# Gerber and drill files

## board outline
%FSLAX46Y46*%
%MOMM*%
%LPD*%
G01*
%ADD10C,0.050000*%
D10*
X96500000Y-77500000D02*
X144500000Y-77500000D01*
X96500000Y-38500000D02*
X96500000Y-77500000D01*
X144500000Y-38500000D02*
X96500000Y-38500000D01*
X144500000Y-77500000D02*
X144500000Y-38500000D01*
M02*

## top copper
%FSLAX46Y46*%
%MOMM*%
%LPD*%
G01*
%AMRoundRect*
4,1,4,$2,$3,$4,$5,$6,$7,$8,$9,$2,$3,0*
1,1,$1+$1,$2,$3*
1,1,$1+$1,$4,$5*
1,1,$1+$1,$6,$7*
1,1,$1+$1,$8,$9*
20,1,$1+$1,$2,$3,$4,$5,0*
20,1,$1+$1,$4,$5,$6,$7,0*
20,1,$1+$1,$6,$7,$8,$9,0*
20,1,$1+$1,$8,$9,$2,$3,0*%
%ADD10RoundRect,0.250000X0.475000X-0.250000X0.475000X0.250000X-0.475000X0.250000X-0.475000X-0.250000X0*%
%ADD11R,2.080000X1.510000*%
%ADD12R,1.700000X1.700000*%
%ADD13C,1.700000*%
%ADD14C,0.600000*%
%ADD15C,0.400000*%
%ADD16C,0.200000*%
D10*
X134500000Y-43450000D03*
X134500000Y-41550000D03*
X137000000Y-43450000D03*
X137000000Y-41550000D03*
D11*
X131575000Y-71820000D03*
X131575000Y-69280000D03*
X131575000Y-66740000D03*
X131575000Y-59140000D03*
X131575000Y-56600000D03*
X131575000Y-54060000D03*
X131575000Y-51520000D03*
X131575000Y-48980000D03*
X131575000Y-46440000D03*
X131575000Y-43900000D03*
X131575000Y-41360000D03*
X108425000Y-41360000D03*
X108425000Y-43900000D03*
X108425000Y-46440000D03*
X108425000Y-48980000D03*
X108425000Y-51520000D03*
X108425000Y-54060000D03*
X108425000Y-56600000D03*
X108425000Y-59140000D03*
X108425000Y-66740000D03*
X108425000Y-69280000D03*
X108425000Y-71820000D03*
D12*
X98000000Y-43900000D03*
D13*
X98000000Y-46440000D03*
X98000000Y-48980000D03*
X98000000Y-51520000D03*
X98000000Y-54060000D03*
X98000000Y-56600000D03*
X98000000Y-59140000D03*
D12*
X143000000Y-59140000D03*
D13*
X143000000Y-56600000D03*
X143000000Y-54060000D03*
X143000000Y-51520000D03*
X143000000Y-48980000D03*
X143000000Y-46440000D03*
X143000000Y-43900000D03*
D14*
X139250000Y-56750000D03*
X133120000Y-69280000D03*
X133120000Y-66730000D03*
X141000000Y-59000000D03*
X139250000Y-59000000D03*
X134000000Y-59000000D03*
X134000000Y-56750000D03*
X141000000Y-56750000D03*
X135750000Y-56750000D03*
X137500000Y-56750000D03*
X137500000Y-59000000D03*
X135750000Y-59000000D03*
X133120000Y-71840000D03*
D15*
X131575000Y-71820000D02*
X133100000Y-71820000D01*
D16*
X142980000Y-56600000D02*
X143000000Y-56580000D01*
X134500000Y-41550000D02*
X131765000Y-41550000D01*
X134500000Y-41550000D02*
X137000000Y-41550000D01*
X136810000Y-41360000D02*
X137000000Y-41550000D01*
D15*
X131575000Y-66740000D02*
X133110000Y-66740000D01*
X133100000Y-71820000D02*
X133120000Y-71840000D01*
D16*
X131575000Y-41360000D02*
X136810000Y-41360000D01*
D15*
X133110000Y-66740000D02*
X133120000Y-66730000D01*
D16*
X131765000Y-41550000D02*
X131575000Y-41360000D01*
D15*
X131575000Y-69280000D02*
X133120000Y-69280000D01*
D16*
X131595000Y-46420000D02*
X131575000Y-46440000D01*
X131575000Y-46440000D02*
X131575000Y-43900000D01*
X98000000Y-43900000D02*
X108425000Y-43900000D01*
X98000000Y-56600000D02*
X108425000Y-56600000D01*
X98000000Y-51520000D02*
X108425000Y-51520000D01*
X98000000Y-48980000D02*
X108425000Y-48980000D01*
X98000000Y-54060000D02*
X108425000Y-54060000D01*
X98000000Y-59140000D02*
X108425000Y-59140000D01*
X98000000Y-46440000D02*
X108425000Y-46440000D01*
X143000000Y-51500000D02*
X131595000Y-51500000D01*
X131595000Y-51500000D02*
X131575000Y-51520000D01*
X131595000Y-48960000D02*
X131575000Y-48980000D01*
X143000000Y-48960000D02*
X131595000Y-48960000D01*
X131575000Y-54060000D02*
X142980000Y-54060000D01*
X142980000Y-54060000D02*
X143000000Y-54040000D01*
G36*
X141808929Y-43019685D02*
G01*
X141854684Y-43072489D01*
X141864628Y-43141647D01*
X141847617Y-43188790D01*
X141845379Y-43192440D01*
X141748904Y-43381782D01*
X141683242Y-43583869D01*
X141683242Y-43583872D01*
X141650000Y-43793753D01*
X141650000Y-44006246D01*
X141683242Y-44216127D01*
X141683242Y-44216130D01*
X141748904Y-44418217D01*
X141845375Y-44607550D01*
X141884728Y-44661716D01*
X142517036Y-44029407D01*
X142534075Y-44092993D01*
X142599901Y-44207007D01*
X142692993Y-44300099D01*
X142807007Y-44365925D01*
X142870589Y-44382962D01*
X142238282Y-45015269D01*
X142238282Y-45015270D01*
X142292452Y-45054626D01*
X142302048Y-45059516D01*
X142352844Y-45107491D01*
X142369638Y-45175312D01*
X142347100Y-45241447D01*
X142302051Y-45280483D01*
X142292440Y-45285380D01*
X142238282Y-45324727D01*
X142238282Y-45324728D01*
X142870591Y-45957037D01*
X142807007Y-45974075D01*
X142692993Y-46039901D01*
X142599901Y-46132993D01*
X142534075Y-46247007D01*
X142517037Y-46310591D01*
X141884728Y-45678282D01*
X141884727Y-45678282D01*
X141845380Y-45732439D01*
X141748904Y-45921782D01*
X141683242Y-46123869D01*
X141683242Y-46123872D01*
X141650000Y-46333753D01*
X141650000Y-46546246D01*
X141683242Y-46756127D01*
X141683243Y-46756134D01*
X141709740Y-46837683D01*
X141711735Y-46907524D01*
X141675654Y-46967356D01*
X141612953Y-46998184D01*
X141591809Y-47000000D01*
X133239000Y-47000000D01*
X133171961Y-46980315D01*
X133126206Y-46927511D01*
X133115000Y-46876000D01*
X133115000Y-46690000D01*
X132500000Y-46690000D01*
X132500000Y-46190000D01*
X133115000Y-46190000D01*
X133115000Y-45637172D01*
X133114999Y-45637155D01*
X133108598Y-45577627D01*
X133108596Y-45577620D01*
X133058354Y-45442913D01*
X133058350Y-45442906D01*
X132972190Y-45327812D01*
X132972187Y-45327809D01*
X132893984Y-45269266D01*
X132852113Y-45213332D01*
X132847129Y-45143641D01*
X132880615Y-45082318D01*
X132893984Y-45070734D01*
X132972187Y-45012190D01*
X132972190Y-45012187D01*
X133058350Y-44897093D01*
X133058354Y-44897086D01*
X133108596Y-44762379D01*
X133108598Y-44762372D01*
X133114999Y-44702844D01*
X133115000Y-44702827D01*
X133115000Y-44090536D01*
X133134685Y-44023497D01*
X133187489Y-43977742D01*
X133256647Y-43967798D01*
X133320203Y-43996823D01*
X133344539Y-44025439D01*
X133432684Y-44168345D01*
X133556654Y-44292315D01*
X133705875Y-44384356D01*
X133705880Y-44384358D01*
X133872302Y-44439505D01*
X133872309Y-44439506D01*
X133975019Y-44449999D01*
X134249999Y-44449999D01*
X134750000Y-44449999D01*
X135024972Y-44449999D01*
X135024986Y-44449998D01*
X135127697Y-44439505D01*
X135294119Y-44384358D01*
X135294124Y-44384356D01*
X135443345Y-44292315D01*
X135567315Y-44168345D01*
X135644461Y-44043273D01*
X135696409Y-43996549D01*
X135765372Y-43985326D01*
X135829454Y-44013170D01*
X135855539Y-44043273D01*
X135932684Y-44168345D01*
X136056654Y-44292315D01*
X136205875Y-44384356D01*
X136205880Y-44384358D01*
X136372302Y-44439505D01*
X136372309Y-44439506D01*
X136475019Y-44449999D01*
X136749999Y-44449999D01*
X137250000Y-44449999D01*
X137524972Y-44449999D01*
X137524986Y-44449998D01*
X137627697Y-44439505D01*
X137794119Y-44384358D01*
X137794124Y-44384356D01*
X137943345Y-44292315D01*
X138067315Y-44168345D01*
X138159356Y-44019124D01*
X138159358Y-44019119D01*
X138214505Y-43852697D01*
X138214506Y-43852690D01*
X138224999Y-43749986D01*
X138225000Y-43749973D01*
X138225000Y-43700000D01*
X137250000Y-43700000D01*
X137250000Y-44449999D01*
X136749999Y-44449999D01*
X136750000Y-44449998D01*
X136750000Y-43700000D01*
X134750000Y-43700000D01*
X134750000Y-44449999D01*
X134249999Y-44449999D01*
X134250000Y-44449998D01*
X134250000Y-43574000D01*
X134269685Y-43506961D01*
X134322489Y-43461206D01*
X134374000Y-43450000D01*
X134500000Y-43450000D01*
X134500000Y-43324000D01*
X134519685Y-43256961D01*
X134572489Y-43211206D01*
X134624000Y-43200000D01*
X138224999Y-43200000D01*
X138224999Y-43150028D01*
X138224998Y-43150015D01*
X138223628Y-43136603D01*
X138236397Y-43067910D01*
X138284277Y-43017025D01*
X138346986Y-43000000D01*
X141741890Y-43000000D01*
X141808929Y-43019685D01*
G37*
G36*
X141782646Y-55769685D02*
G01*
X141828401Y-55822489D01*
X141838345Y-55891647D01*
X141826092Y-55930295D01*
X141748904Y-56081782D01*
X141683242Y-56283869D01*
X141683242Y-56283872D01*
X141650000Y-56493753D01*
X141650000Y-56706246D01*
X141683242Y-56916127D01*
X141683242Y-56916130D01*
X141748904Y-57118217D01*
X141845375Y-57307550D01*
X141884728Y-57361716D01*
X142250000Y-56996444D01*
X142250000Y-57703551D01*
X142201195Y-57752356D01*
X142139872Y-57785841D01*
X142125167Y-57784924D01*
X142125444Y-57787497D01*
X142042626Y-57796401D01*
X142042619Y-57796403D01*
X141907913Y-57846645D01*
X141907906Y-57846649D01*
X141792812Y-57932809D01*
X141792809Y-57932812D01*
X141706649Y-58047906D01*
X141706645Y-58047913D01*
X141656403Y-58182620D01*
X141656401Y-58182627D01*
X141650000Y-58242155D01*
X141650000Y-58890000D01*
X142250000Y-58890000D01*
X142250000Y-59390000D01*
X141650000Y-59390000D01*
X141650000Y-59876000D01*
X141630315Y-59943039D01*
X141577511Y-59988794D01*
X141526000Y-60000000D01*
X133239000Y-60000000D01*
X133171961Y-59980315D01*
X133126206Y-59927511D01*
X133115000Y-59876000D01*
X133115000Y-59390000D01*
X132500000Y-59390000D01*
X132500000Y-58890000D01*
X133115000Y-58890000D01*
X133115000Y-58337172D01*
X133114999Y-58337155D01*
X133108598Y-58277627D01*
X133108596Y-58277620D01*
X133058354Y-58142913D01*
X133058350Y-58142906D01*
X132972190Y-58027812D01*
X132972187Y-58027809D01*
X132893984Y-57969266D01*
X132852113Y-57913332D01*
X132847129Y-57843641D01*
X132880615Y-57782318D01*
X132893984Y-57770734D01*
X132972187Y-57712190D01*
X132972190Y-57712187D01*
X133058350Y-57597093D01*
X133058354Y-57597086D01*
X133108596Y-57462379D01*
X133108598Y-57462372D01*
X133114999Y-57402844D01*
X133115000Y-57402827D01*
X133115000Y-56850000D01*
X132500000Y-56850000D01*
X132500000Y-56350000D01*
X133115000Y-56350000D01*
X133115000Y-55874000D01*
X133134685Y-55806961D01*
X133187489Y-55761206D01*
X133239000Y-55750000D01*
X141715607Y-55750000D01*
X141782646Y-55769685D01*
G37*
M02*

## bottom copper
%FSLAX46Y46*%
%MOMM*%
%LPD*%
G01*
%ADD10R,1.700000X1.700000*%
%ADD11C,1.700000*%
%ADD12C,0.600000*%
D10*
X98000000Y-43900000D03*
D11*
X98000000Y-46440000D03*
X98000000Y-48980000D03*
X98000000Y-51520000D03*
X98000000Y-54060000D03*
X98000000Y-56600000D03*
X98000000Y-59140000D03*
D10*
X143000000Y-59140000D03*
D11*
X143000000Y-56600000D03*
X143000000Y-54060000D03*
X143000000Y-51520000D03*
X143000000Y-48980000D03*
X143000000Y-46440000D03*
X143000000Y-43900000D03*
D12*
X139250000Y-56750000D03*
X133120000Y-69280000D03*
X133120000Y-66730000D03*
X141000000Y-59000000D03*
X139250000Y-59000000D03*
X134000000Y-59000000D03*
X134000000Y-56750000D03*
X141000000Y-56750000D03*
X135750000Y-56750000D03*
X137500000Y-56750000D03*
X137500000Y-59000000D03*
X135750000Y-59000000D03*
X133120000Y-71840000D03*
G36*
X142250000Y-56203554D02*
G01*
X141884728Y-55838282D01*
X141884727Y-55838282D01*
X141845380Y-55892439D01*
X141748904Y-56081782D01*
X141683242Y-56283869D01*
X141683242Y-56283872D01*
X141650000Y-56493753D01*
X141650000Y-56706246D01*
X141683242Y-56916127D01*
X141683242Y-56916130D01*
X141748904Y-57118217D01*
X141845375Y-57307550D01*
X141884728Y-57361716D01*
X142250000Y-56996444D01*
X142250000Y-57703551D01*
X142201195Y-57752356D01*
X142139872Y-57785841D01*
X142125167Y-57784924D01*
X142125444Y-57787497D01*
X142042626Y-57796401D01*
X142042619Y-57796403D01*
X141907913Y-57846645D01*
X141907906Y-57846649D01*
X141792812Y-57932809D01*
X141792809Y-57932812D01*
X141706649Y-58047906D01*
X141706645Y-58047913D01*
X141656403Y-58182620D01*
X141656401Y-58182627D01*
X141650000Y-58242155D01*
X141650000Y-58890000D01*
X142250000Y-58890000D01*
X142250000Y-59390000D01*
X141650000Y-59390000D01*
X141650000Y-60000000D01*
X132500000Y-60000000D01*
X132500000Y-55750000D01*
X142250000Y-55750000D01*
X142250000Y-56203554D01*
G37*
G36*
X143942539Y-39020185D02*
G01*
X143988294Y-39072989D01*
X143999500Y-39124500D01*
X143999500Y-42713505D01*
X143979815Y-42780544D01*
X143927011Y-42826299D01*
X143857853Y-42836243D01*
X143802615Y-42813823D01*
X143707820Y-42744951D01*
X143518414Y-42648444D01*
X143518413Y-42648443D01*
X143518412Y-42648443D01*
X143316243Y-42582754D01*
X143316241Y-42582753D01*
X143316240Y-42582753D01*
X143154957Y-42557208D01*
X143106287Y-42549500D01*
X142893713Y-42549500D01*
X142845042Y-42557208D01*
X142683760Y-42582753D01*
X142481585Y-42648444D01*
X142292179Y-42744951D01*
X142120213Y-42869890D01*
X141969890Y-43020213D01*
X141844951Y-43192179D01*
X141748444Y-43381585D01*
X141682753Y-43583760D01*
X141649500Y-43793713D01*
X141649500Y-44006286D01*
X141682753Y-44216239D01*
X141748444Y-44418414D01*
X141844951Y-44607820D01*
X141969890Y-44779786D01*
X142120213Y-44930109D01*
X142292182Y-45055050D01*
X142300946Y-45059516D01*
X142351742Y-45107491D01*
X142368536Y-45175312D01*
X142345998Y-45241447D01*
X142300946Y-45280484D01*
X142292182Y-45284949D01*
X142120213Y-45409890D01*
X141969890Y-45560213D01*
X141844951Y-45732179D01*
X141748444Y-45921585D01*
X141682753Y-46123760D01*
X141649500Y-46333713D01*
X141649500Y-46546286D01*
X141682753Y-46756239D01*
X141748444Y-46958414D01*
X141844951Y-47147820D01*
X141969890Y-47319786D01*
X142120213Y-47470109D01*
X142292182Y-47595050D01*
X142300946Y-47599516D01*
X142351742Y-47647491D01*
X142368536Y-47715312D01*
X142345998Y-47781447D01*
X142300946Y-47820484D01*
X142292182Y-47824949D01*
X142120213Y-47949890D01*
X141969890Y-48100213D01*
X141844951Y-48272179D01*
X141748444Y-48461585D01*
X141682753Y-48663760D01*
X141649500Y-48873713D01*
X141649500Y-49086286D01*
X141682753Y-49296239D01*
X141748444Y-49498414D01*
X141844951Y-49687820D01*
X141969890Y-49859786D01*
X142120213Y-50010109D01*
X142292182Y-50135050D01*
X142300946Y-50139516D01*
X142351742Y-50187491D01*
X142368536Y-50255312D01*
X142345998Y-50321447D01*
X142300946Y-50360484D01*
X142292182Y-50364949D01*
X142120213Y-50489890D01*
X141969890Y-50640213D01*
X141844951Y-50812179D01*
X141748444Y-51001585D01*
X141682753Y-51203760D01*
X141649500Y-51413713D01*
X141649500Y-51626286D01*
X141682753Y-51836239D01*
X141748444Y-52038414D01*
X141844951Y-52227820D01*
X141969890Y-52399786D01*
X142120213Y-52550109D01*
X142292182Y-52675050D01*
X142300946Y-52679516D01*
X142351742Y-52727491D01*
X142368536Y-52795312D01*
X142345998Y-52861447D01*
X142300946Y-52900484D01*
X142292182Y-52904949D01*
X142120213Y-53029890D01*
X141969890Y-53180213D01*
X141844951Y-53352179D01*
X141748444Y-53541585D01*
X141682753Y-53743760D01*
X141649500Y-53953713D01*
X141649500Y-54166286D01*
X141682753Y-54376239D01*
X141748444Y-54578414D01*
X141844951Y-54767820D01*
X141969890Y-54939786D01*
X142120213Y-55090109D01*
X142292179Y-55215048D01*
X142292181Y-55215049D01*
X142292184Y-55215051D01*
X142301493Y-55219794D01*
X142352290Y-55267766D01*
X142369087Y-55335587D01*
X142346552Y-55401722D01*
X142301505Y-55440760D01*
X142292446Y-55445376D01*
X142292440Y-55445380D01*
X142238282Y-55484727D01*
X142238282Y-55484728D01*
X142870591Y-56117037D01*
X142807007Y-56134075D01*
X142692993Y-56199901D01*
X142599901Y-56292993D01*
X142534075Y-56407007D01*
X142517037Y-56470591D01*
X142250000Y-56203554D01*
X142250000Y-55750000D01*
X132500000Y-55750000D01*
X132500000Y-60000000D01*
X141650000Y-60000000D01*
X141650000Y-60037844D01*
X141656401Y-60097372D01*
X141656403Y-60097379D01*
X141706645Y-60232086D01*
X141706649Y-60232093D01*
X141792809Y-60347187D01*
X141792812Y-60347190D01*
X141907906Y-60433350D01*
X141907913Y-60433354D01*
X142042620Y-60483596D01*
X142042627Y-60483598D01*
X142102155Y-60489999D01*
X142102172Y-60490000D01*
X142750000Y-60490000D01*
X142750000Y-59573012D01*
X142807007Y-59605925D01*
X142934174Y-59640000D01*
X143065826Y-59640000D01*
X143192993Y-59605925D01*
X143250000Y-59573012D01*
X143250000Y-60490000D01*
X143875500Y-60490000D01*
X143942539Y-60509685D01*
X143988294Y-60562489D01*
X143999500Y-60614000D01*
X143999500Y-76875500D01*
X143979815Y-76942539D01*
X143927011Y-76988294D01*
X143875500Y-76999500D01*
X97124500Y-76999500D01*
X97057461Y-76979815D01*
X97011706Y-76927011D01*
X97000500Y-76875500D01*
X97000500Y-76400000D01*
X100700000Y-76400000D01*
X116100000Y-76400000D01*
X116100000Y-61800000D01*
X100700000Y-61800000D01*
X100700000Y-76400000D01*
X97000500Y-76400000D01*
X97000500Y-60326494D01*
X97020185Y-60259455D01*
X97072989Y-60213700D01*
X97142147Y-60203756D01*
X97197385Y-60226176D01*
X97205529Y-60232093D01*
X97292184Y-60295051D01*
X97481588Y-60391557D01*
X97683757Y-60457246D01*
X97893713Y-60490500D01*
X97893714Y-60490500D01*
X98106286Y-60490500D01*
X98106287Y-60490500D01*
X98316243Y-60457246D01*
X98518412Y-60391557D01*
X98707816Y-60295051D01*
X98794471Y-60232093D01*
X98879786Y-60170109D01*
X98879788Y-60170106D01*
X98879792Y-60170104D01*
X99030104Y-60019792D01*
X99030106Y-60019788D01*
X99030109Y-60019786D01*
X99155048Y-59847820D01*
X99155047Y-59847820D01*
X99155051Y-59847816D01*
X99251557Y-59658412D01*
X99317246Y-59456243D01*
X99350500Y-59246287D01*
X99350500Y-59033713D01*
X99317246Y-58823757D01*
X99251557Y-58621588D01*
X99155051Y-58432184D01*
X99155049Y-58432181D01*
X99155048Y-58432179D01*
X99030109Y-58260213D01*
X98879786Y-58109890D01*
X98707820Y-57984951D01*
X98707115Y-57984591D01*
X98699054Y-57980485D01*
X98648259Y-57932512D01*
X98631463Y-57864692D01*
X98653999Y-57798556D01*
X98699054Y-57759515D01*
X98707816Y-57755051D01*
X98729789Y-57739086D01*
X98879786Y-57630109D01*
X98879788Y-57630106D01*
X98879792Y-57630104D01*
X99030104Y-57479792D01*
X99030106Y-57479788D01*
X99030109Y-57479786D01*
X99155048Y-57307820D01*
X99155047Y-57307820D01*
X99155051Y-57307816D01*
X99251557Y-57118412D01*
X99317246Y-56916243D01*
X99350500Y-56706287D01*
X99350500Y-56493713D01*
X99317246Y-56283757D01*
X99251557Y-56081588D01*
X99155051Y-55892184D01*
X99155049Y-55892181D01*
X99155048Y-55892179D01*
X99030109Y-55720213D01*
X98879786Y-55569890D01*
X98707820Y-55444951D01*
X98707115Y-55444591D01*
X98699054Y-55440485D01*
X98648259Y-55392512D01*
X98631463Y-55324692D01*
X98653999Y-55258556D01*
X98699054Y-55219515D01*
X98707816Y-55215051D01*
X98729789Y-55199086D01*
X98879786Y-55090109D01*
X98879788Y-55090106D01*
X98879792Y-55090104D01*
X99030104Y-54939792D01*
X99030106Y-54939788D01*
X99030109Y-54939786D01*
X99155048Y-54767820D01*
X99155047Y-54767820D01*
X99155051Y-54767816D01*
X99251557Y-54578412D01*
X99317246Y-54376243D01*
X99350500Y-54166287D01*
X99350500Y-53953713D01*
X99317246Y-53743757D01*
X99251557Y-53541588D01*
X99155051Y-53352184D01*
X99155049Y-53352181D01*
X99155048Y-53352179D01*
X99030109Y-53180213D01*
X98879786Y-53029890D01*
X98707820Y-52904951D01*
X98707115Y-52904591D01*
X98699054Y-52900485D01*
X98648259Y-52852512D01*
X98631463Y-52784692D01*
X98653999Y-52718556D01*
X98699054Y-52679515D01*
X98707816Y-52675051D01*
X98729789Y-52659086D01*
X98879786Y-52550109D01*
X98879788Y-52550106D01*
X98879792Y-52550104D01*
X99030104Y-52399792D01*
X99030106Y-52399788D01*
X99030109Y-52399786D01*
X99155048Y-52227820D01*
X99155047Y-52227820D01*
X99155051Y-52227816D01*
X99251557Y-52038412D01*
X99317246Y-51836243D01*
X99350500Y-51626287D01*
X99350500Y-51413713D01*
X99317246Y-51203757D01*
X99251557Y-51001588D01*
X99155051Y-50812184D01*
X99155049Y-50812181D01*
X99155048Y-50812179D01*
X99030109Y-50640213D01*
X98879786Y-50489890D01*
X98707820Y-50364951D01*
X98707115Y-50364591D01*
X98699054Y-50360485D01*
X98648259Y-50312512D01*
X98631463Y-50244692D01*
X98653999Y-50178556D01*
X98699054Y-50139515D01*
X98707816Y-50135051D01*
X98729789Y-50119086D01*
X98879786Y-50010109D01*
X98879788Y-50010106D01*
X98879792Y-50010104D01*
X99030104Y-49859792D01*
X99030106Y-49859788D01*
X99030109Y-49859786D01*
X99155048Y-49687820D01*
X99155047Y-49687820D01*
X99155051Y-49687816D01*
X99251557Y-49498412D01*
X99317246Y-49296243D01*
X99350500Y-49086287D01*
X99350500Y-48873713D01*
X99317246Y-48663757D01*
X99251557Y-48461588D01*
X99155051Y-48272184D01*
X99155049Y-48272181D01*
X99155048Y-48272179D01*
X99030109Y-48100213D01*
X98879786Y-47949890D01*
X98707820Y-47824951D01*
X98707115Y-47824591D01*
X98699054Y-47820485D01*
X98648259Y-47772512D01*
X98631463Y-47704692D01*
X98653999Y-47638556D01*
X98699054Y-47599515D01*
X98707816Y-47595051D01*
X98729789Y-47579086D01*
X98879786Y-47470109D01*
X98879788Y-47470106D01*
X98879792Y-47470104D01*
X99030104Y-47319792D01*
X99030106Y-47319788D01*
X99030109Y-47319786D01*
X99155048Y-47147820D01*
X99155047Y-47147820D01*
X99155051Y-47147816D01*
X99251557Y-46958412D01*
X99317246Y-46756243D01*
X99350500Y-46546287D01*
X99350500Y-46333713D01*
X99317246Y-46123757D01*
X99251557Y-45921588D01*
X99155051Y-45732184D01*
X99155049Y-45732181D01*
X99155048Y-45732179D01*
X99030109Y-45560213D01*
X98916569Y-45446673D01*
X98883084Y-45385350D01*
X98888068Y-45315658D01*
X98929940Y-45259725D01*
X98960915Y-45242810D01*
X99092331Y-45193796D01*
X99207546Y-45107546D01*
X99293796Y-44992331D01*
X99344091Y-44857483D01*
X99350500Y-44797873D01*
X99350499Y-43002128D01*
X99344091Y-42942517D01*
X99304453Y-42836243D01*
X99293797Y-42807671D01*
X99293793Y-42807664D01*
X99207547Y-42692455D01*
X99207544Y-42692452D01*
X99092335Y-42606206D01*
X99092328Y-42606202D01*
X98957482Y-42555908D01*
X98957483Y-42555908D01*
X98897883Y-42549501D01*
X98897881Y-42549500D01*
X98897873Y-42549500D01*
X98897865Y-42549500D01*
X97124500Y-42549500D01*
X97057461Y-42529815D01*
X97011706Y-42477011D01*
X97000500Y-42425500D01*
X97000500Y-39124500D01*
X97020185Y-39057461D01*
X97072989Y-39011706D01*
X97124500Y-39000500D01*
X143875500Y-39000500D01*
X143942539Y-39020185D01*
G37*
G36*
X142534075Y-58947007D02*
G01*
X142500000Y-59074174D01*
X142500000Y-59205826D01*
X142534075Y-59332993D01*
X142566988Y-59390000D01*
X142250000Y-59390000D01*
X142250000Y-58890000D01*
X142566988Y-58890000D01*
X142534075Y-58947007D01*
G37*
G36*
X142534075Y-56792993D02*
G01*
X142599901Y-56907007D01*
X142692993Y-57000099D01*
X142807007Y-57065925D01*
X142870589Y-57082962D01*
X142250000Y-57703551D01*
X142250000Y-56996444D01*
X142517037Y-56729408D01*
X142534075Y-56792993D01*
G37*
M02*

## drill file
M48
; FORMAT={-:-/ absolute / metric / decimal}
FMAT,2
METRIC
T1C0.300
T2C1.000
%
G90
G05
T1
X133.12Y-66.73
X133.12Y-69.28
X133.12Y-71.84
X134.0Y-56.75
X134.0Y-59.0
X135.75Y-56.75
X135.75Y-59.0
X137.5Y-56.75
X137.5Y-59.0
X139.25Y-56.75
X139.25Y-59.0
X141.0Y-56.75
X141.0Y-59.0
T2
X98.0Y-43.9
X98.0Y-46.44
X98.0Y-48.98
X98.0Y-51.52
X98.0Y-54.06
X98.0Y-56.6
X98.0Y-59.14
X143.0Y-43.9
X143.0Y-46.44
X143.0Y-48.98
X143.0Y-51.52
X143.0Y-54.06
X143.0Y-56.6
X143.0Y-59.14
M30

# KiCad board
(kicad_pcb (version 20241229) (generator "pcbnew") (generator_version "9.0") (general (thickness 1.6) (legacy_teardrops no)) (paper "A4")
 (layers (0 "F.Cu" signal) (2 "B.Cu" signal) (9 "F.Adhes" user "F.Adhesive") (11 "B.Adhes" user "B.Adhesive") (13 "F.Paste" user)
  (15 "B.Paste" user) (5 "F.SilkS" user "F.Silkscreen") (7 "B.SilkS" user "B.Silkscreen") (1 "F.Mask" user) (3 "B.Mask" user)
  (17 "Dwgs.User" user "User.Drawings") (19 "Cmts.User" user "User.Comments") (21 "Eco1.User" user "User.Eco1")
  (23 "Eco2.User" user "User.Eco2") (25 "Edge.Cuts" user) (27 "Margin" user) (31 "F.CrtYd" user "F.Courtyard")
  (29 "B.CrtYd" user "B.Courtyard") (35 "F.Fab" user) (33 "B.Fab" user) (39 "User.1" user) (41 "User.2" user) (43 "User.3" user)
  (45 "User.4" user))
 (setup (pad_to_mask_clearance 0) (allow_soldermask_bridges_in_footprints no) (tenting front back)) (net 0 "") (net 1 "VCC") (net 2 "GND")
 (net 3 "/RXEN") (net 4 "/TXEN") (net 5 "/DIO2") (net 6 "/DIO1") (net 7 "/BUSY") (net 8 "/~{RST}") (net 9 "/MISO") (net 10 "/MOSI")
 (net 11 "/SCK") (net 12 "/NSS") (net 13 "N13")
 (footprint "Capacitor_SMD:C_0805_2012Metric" (layer "F.Cu") (at 134.5 42.5 90)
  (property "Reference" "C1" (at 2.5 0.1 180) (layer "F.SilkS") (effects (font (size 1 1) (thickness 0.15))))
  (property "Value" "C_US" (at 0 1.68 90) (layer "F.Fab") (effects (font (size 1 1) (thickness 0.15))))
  (pad "1" smd roundrect (at -0.95 0 90) (size 1 1.45) (layers "F.Cu" "F.Mask" "F.Paste") (roundrect_rratio 0.25) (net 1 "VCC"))
  (pad "2" smd roundrect (at 0.95 0 90) (size 1 1.45) (layers "F.Cu" "F.Mask" "F.Paste") (roundrect_rratio 0.25) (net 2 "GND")))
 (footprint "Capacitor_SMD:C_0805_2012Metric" (layer "F.Cu") (at 137 42.5 90)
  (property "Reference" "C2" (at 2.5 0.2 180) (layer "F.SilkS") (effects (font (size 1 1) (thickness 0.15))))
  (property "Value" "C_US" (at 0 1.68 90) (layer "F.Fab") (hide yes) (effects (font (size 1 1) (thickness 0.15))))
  (pad "1" smd roundrect (at -0.95 0 90) (size 1 1.45) (layers "F.Cu" "F.Mask" "F.Paste") (roundrect_rratio 0.25) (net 1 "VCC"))
  (pad "2" smd roundrect (at 0.95 0 90) (size 1 1.45) (layers "F.Cu" "F.Mask" "F.Paste") (roundrect_rratio 0.25) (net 2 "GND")))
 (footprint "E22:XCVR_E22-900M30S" (layer "F.Cu") (at 120 58)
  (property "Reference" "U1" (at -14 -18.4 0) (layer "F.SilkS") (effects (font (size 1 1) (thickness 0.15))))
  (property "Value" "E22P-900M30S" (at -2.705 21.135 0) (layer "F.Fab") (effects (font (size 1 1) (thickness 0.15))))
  (pad "1" smd rect (at 11.575 13.82) (size 2.08 1.51) (layers "F.Cu" "F.Mask" "F.Paste") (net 2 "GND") (solder_mask_margin 0.102))
  (pad "2" smd rect (at 11.575 11.28) (size 2.08 1.51) (layers "F.Cu" "F.Mask" "F.Paste") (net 2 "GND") (solder_mask_margin 0.102))
  (pad "3" smd rect (at 11.575 8.74) (size 2.08 1.51) (layers "F.Cu" "F.Mask" "F.Paste") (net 2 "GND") (solder_mask_margin 0.102))
  (pad "4" smd rect (at 11.575 1.14) (size 2.08 1.51) (layers "F.Cu" "F.Mask" "F.Paste") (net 2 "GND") (solder_mask_margin 0.102))
  (pad "5" smd rect (at 11.575 -1.4) (size 2.08 1.51) (layers "F.Cu" "F.Mask" "F.Paste") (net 2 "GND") (solder_mask_margin 0.102))
  (pad "6" smd rect (at 11.575 -3.94) (size 2.08 1.51) (layers "F.Cu" "F.Mask" "F.Paste") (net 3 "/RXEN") (solder_mask_margin 0.102))
  (pad "7" smd rect (at 11.575 -6.48) (size 2.08 1.51) (layers "F.Cu" "F.Mask" "F.Paste") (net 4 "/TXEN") (solder_mask_margin 0.102))
  (pad "8" smd rect (at 11.575 -9.02) (size 2.08 1.51) (layers "F.Cu" "F.Mask" "F.Paste") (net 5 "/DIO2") (solder_mask_margin 0.102))
  (pad "9" smd rect (at 11.575 -11.56) (size 2.08 1.51) (layers "F.Cu" "F.Mask" "F.Paste") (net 1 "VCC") (solder_mask_margin 0.102))
  (pad "10" smd rect (at 11.575 -14.1) (size 2.08 1.51) (layers "F.Cu" "F.Mask" "F.Paste") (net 1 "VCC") (solder_mask_margin 0.102))
  (pad "11" smd rect (at 11.575 -16.64) (size 2.08 1.51) (layers "F.Cu" "F.Mask" "F.Paste") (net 2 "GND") (solder_mask_margin 0.102))
  (pad "12" smd rect (at -11.575 -16.64) (size 2.08 1.51) (layers "F.Cu" "F.Mask" "F.Paste") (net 2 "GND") (solder_mask_margin 0.102))
  (pad "13" smd rect (at -11.575 -14.1) (size 2.08 1.51) (layers "F.Cu" "F.Mask" "F.Paste") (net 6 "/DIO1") (solder_mask_margin 0.102))
  (pad "14" smd rect (at -11.575 -11.56) (size 2.08 1.51) (layers "F.Cu" "F.Mask" "F.Paste") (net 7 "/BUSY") (solder_mask_margin 0.102))
  (pad "15" smd rect (at -11.575 -9.02) (size 2.08 1.51) (layers "F.Cu" "F.Mask" "F.Paste") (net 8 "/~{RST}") (solder_mask_margin 0.102))
  (pad "16" smd rect (at -11.575 -6.48) (size 2.08 1.51) (layers "F.Cu" "F.Mask" "F.Paste") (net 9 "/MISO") (solder_mask_margin 0.102))
  (pad "17" smd rect (at -11.575 -3.94) (size 2.08 1.51) (layers "F.Cu" "F.Mask" "F.Paste") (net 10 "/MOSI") (solder_mask_margin 0.102))
  (pad "18" smd rect (at -11.575 -1.4) (size 2.08 1.51) (layers "F.Cu" "F.Mask" "F.Paste") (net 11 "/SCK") (solder_mask_margin 0.102))
  (pad "19" smd rect (at -11.575 1.14) (size 2.08 1.51) (layers "F.Cu" "F.Mask" "F.Paste") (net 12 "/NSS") (solder_mask_margin 0.102))
  (pad "20" smd rect (at -11.575 8.74) (size 2.08 1.51) (layers "F.Cu" "F.Mask" "F.Paste") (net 2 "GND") (solder_mask_margin 0.102))
  (pad "21" smd rect (at -11.575 11.28) (size 2.08 1.51) (layers "F.Cu" "F.Mask" "F.Paste") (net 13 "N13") (solder_mask_margin 0.102))
  (pad "22" smd rect (at -11.575 13.82) (size 2.08 1.51) (layers "F.Cu" "F.Mask" "F.Paste") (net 2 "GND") (solder_mask_margin 0.102)))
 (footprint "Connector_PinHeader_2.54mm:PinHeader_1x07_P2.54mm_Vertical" (layer "B.Cu") (at 98 43.9 180)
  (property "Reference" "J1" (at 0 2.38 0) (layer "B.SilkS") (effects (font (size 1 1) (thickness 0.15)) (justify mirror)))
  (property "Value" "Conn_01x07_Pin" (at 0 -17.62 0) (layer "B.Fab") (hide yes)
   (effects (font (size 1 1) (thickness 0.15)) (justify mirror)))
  (pad "1" thru_hole rect (at 0 0 180) (size 1.7 1.7) (drill 1) (layers "*.Cu" "*.Mask") (remove_unused_layers no) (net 6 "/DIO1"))
  (pad "2" thru_hole circle (at 0 -2.54 180) (size 1.7 1.7) (drill 1) (layers "*.Cu" "*.Mask") (remove_unused_layers no) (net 7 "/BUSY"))
  (pad "3" thru_hole circle (at 0 -5.08 180) (size 1.7 1.7) (drill 1) (layers "*.Cu" "*.Mask") (remove_unused_layers no) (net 8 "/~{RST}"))
  (pad "4" thru_hole circle (at 0 -7.62 180) (size 1.7 1.7) (drill 1) (layers "*.Cu" "*.Mask") (remove_unused_layers no) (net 9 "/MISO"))
  (pad "5" thru_hole circle (at 0 -10.16 180) (size 1.7 1.7) (drill 1) (layers "*.Cu" "*.Mask") (remove_unused_layers no) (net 10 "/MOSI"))
  (pad "6" thru_hole circle (at 0 -12.7 180) (size 1.7 1.7) (drill 1) (layers "*.Cu" "*.Mask") (remove_unused_layers no) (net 11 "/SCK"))
  (pad "7" thru_hole circle (at 0 -15.24 180) (size 1.7 1.7) (drill 1) (layers "*.Cu" "*.Mask") (remove_unused_layers no) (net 12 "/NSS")))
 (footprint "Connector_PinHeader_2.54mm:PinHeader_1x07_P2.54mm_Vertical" (layer "B.Cu") (at 143 59.14)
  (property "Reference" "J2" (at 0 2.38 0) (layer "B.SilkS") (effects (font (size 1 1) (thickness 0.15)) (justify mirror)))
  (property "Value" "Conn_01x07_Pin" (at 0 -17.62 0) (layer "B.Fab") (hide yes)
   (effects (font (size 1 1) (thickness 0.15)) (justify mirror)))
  (pad "1" thru_hole rect (at 0 0) (size 1.7 1.7) (drill 1) (layers "*.Cu" "*.Mask") (remove_unused_layers no) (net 2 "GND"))
  (pad "2" thru_hole circle (at 0 -2.54) (size 1.7 1.7) (drill 1) (layers "*.Cu" "*.Mask") (remove_unused_layers no) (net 2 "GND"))
  (pad "3" thru_hole circle (at 0 -5.08) (size 1.7 1.7) (drill 1) (layers "*.Cu" "*.Mask") (remove_unused_layers no) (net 3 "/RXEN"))
  (pad "4" thru_hole circle (at 0 -7.62) (size 1.7 1.7) (drill 1) (layers "*.Cu" "*.Mask") (remove_unused_layers no) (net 4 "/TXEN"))
  (pad "5" thru_hole circle (at 0 -10.16) (size 1.7 1.7) (drill 1) (layers "*.Cu" "*.Mask") (remove_unused_layers no) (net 5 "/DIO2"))
  (pad "6" thru_hole circle (at 0 -12.7) (size 1.7 1.7) (drill 1) (layers "*.Cu" "*.Mask") (remove_unused_layers no) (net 1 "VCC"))
  (pad "7" thru_hole circle (at 0 -15.24) (size 1.7 1.7) (drill 1) (layers "*.Cu" "*.Mask") (remove_unused_layers no) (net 1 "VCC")))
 (gr_line (start 96.5 77.5) (end 144.5 77.5) (stroke (width 0.05) (type default)) (layer "Edge.Cuts"))
 (gr_line (start 96.5 38.5) (end 96.5 77.5) (stroke (width 0.05) (type default)) (layer "Edge.Cuts"))
 (gr_line (start 144.5 38.5) (end 96.5 38.5) (stroke (width 0.05) (type default)) (layer "Edge.Cuts"))
 (gr_line (start 144.5 77.5) (end 144.5 38.5) (stroke (width 0.05) (type default)) (layer "Edge.Cuts"))
 (segment (start 131.575 71.82) (end 133.1 71.82) (width 0.4) (layer "F.Cu") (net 2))
 (segment (start 142.98 56.6) (end 143 56.58) (width 0.2) (layer "F.Cu") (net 2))
 (segment (start 134.5 41.55) (end 131.765 41.55) (width 0.2) (layer "F.Cu") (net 2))
 (segment (start 134.5 41.55) (end 137 41.55) (width 0.2) (layer "F.Cu") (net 2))
 (segment (start 136.81 41.36) (end 137 41.55) (width 0.2) (layer "F.Cu") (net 2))
 (segment (start 131.575 66.74) (end 133.11 66.74) (width 0.4) (layer "F.Cu") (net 2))
 (segment (start 133.1 71.82) (end 133.12 71.84) (width 0.4) (layer "F.Cu") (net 2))
 (segment (start 131.575 41.36) (end 136.81 41.36) (width 0.2) (layer "F.Cu") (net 2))
 (segment (start 133.11 66.74) (end 133.12 66.73) (width 0.4) (layer "F.Cu") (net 2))
 (segment (start 131.765 41.55) (end 131.575 41.36) (width 0.2) (layer "F.Cu") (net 2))
 (segment (start 131.575 69.28) (end 133.12 69.28) (width 0.4) (layer "F.Cu") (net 2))
 (via (at 139.25 56.75) (size 0.6) (drill 0.3) (layers "F.Cu" "B.Cu") (free yes) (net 2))
 (via (at 133.12 69.28) (size 0.6) (drill 0.3) (layers "F.Cu" "B.Cu") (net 2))
 (via (at 133.12 66.73) (size 0.6) (drill 0.3) (layers "F.Cu" "B.Cu") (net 2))
 (via (at 141 59) (size 0.6) (drill 0.3) (layers "F.Cu" "B.Cu") (free yes) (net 2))
 (via (at 139.25 59) (size 0.6) (drill 0.3) (layers "F.Cu" "B.Cu") (free yes) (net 2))
 (via (at 134 59) (size 0.6) (drill 0.3) (layers "F.Cu" "B.Cu") (free yes) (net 2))
 (via (at 134 56.75) (size 0.6) (drill 0.3) (layers "F.Cu" "B.Cu") (free yes) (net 2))
 (via (at 141 56.75) (size 0.6) (drill 0.3) (layers "F.Cu" "B.Cu") (free yes) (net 2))
 (via (at 135.75 56.75) (size 0.6) (drill 0.3) (layers "F.Cu" "B.Cu") (free yes) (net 2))
 (via (at 137.5 56.75) (size 0.6) (drill 0.3) (layers "F.Cu" "B.Cu") (free yes) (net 2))
 (via (at 137.5 59) (size 0.6) (drill 0.3) (layers "F.Cu" "B.Cu") (free yes) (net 2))
 (via (at 135.75 59) (size 0.6) (drill 0.3) (layers "F.Cu" "B.Cu") (free yes) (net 2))
 (via (at 133.12 71.84) (size 0.6) (drill 0.3) (layers "F.Cu" "B.Cu") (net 2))
 (segment (start 131.595 46.42) (end 131.575 46.44) (width 0.2) (layer "F.Cu") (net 1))
 (segment (start 131.575 46.44) (end 131.575 43.9) (width 0.2) (layer "F.Cu") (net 1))
 (segment (start 98 43.9) (end 108.425 43.9) (width 0.2) (layer "F.Cu") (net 6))
 (segment (start 98 56.6) (end 108.425 56.6) (width 0.2) (layer "F.Cu") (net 11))
 (segment (start 98 51.52) (end 108.425 51.52) (width 0.2) (layer "F.Cu") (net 9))
 (segment (start 98 48.98) (end 108.425 48.98) (width 0.2) (layer "F.Cu") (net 8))
 (segment (start 98 54.06) (end 108.425 54.06) (width 0.2) (layer "F.Cu") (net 10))
 (segment (start 98 59.14) (end 108.425 59.14) (width 0.2) (layer "F.Cu") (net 12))
 (segment (start 98 46.44) (end 108.425 46.44) (width 0.2) (layer "F.Cu") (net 7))
 (segment (start 143 51.5) (end 131.595 51.5) (width 0.2) (layer "F.Cu") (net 4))
 (segment (start 131.595 51.5) (end 131.575 51.52) (width 0.2) (layer "F.Cu") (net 4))
 (segment (start 131.595 48.96) (end 131.575 48.98) (width 0.2) (layer "F.Cu") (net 5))
 (segment (start 143 48.96) (end 131.595 48.96) (width 0.2) (layer "F.Cu") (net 5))
 (segment (start 131.575 54.06) (end 142.98 54.06) (width 0.2) (layer "F.Cu") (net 3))
 (segment (start 142.98 54.06) (end 143 54.04) (width 0.2) (layer "F.Cu") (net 3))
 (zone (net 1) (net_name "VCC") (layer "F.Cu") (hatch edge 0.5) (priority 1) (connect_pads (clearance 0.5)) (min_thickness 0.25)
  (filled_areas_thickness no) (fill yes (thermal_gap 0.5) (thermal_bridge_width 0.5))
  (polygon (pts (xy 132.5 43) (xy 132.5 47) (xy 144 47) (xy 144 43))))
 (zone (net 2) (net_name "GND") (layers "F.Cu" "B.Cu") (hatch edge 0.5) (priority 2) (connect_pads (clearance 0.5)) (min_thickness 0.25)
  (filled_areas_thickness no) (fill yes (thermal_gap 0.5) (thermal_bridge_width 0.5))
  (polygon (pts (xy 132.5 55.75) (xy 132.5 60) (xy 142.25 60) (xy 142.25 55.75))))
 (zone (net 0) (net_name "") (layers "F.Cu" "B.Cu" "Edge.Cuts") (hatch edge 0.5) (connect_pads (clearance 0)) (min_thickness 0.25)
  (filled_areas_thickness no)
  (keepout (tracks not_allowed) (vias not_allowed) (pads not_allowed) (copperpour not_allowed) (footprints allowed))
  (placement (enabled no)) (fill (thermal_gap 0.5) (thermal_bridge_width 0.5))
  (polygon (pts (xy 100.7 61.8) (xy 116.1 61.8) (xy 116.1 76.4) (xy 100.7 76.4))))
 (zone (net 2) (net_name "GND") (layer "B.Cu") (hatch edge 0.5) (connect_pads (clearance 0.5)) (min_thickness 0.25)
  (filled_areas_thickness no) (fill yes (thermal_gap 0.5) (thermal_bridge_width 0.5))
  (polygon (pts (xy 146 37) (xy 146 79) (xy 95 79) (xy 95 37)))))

